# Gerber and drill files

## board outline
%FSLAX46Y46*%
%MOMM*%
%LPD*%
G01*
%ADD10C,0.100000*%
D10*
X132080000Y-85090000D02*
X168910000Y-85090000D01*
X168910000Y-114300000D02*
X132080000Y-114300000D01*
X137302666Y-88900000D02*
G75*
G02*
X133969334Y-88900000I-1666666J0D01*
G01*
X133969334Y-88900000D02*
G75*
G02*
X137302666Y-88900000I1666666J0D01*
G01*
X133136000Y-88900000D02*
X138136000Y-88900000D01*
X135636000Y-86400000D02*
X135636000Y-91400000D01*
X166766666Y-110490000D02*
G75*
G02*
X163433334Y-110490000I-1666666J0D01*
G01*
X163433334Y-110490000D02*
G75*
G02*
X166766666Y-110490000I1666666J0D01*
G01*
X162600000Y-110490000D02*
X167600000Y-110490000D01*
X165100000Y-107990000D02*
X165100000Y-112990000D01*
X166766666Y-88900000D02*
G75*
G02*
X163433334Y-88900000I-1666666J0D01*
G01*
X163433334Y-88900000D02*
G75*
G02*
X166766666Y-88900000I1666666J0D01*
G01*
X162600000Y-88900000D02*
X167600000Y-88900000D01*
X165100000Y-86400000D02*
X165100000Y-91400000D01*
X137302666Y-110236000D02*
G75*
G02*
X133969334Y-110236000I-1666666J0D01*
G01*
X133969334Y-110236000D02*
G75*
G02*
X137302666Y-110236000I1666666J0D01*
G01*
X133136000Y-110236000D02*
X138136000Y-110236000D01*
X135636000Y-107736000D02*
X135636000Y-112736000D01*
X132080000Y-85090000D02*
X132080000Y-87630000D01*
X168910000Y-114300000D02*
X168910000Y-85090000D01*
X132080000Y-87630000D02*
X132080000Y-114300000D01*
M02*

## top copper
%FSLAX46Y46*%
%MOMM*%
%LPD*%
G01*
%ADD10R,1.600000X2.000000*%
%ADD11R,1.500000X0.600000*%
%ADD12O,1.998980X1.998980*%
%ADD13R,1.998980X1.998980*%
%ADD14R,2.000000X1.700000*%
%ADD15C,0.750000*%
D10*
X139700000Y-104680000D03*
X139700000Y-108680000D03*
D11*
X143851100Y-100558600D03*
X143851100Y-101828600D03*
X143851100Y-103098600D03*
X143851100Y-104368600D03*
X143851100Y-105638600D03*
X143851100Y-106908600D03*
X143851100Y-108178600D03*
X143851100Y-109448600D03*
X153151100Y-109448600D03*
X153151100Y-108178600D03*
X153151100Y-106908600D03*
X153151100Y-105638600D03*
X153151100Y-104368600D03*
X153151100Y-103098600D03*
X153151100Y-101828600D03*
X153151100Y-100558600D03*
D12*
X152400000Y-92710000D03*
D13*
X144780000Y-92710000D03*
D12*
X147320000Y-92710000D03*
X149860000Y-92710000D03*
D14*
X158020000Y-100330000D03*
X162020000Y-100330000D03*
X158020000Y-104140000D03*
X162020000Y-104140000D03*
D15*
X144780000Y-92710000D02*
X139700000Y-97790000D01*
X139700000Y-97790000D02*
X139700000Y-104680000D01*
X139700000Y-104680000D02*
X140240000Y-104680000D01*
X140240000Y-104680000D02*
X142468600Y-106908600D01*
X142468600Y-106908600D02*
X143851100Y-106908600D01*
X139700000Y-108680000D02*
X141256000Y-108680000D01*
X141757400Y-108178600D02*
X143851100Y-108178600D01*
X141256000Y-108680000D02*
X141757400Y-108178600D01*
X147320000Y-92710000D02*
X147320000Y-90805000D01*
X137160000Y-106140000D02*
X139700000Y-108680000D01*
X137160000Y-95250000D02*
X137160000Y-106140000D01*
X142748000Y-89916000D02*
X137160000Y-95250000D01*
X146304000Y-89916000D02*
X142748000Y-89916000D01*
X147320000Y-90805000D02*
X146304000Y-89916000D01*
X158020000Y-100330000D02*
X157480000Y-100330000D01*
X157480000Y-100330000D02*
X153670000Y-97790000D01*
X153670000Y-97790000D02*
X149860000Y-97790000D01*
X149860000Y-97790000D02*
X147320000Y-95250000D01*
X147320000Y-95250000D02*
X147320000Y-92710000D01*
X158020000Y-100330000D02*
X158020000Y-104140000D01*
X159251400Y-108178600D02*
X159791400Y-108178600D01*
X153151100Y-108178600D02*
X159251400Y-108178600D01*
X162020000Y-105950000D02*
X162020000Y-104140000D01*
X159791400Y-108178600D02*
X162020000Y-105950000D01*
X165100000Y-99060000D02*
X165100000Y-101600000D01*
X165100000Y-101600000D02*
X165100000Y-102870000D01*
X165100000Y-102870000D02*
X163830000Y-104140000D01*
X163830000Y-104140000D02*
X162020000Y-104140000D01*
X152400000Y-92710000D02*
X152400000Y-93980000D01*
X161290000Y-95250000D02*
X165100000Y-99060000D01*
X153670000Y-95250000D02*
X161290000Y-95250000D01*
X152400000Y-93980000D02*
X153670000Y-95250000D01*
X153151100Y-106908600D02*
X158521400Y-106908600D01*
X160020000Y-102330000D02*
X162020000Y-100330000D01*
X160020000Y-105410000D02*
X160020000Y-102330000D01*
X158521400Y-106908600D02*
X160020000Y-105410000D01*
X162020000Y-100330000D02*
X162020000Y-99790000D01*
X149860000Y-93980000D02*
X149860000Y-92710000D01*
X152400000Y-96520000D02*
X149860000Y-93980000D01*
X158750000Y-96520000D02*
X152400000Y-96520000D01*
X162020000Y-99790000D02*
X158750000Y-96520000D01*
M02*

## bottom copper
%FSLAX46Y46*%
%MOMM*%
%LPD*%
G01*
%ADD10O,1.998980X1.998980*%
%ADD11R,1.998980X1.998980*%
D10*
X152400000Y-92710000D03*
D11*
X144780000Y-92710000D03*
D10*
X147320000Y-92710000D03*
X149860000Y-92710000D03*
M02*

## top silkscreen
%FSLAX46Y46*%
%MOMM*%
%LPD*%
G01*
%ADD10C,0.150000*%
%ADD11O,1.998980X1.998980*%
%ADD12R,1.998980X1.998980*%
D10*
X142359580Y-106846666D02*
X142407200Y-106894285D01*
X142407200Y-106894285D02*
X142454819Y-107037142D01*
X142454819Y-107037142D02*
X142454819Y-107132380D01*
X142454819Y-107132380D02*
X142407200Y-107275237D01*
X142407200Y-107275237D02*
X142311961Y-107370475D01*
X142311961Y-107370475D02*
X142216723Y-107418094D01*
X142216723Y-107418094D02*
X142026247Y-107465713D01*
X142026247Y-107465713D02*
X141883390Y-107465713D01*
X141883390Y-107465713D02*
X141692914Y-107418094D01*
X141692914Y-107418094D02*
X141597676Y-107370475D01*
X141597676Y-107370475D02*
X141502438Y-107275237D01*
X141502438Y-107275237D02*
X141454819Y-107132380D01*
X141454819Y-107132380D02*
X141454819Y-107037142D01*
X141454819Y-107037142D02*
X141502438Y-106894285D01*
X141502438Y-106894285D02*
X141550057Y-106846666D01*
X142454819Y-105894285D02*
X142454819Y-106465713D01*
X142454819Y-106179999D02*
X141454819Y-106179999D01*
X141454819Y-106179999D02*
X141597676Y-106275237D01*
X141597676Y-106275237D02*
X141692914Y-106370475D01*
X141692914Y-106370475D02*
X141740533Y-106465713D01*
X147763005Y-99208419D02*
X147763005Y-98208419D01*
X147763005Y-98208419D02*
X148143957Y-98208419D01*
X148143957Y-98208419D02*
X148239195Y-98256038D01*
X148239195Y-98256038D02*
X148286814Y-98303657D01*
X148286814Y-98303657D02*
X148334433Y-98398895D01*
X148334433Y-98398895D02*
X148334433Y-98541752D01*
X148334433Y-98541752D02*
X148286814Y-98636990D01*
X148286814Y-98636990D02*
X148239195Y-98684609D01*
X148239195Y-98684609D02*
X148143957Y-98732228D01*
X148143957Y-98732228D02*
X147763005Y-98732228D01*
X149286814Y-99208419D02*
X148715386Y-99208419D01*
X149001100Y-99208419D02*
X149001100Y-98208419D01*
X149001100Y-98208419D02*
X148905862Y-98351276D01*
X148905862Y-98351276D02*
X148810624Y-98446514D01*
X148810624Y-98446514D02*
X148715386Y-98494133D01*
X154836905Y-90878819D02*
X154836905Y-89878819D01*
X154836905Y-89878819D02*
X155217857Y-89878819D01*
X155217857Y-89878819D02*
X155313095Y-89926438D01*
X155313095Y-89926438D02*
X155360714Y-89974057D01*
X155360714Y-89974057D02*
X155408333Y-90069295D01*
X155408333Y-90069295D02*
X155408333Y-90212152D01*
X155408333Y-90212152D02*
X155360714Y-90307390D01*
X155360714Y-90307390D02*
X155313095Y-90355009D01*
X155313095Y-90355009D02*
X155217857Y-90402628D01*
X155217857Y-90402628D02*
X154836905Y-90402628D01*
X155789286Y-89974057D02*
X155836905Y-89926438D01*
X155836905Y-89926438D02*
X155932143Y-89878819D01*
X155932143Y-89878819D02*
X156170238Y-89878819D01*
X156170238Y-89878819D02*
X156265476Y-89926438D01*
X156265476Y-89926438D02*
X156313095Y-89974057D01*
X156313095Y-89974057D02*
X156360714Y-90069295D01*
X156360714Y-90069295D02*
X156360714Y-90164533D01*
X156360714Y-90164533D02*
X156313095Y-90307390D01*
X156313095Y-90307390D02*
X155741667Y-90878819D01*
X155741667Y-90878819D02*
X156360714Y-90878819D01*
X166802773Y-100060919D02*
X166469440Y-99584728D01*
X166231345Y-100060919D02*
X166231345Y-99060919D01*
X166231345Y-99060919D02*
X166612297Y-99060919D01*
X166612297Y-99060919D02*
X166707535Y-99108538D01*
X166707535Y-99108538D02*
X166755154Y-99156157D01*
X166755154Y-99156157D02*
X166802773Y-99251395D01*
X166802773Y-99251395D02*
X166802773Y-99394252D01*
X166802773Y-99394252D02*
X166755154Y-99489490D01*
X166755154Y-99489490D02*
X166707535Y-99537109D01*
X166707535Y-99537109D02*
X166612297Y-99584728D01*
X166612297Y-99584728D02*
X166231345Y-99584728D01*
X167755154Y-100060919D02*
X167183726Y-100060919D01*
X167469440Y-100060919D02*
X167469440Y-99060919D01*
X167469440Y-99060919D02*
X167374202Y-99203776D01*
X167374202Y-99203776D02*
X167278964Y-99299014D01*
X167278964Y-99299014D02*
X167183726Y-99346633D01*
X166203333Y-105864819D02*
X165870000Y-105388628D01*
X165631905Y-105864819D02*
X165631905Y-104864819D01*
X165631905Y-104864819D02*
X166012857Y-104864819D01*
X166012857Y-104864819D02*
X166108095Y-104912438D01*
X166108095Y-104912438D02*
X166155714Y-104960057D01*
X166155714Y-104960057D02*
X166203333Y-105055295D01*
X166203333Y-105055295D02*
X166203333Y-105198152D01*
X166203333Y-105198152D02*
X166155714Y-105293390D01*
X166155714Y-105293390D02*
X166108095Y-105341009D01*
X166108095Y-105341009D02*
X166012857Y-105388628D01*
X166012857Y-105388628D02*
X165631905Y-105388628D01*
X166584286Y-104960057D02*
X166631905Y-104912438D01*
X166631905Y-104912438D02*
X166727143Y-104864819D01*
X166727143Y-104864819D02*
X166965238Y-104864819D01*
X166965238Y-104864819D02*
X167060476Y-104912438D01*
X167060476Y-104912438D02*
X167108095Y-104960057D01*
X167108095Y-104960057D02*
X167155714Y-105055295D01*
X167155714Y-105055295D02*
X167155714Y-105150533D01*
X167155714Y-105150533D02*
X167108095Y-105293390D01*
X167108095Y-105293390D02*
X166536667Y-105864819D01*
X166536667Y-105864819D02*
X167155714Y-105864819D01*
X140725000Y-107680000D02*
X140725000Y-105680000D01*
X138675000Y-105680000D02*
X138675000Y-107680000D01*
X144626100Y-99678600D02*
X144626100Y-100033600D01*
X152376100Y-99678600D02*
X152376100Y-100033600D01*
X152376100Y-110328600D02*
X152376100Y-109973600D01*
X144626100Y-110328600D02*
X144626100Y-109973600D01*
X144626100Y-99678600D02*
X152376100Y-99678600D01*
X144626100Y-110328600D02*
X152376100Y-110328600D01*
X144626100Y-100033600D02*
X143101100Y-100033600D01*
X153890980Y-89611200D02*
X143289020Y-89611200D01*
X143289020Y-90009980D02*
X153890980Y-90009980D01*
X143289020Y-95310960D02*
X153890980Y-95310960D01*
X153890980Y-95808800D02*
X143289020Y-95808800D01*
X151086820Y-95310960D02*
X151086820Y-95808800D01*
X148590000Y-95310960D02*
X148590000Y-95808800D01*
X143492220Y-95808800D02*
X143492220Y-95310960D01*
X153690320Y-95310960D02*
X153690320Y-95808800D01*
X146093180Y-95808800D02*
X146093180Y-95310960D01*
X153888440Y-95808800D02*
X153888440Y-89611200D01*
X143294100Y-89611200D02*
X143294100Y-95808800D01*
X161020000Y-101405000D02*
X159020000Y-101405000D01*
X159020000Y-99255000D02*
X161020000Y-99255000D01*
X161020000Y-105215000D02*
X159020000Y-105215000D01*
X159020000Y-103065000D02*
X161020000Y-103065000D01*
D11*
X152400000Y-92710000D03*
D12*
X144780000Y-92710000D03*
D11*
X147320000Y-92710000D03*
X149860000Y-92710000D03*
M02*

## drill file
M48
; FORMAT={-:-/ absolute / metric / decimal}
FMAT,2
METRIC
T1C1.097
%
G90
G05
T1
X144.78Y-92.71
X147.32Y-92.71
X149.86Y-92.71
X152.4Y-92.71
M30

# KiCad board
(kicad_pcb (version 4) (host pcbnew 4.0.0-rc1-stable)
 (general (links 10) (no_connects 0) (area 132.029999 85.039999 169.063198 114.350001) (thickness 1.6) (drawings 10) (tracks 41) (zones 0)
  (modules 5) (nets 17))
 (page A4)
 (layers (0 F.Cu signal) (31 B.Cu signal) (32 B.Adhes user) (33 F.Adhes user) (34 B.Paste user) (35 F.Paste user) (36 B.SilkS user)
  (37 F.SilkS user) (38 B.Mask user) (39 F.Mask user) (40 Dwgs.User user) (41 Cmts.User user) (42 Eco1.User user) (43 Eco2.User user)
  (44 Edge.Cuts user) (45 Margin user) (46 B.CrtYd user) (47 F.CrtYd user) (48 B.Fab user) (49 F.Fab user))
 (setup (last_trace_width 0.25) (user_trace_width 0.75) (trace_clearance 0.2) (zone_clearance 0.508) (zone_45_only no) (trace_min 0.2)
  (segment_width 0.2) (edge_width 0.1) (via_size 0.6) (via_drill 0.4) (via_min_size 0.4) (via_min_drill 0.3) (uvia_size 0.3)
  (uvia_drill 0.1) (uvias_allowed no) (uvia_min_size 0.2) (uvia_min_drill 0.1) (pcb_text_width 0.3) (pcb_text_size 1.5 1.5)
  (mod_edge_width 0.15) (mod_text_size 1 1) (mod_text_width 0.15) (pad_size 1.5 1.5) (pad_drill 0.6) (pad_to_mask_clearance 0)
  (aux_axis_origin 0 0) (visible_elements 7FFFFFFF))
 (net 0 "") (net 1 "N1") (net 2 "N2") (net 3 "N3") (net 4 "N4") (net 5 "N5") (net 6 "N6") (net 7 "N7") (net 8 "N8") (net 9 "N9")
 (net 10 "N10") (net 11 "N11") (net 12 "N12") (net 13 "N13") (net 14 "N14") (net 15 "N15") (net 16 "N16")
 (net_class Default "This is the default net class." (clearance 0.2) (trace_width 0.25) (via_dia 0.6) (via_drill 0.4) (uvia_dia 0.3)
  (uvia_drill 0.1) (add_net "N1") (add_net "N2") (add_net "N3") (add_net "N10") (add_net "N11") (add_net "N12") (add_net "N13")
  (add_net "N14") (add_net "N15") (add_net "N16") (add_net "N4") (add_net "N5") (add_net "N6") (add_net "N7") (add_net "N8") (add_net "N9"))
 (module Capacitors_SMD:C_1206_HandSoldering (layer F.Cu) (at 139.7 106.68 270)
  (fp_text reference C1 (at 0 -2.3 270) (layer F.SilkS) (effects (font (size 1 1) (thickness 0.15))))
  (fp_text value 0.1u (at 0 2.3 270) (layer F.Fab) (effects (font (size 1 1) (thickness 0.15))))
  (fp_line (start 1 -1.025) (end -1 -1.025) (layer F.SilkS) (width 0.15))
  (fp_line (start -1 1.025) (end 1 1.025) (layer F.SilkS) (width 0.15))
  (pad 1 smd rect (at -2 0 270) (size 2 1.6) (layers F.Cu F.Paste F.Mask) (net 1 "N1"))
  (pad 2 smd rect (at 2 0 270) (size 2 1.6) (layers F.Cu F.Paste F.Mask) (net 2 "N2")))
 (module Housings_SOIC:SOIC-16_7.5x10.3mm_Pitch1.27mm (layer F.Cu) (at 148.5011 105.0036)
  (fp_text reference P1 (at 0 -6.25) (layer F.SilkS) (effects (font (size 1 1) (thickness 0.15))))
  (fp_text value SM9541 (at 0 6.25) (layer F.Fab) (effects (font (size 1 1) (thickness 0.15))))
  (fp_line (start -3.875 -5.325) (end -3.875 -4.97) (layer F.SilkS) (width 0.15))
  (fp_line (start 3.875 -5.325) (end 3.875 -4.97) (layer F.SilkS) (width 0.15))
  (fp_line (start 3.875 5.325) (end 3.875 4.97) (layer F.SilkS) (width 0.15))
  (fp_line (start -3.875 5.325) (end -3.875 4.97) (layer F.SilkS) (width 0.15))
  (fp_line (start -3.875 -5.325) (end 3.875 -5.325) (layer F.SilkS) (width 0.15))
  (fp_line (start -3.875 5.325) (end 3.875 5.325) (layer F.SilkS) (width 0.15))
  (fp_line (start -3.875 -4.97) (end -5.4 -4.97) (layer F.SilkS) (width 0.15))
  (pad 1 smd rect (at -4.65 -4.445) (size 1.5 0.6) (layers F.Cu F.Paste F.Mask) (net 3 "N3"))
  (pad 2 smd rect (at -4.65 -3.175) (size 1.5 0.6) (layers F.Cu F.Paste F.Mask) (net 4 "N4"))
  (pad 3 smd rect (at -4.65 -1.905) (size 1.5 0.6) (layers F.Cu F.Paste F.Mask) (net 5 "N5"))
  (pad 4 smd rect (at -4.65 -0.635) (size 1.5 0.6) (layers F.Cu F.Paste F.Mask) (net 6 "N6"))
  (pad 5 smd rect (at -4.65 0.635) (size 1.5 0.6) (layers F.Cu F.Paste F.Mask) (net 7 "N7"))
  (pad 6 smd rect (at -4.65 1.905) (size 1.5 0.6) (layers F.Cu F.Paste F.Mask) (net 1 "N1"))
  (pad 7 smd rect (at -4.65 3.175) (size 1.5 0.6) (layers F.Cu F.Paste F.Mask) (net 2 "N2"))
  (pad 8 smd rect (at -4.65 4.445) (size 1.5 0.6) (layers F.Cu F.Paste F.Mask) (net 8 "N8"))
  (pad 9 smd rect (at 4.65 4.445) (size 1.5 0.6) (layers F.Cu F.Paste F.Mask) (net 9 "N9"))
  (pad 10 smd rect (at 4.65 3.175) (size 1.5 0.6) (layers F.Cu F.Paste F.Mask) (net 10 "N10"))
  (pad 11 smd rect (at 4.65 1.905) (size 1.5 0.6) (layers F.Cu F.Paste F.Mask) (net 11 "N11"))
  (pad 12 smd rect (at 4.65 0.635) (size 1.5 0.6) (layers F.Cu F.Paste F.Mask) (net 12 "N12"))
  (pad 13 smd rect (at 4.65 -0.635) (size 1.5 0.6) (layers F.Cu F.Paste F.Mask) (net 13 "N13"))
  (pad 14 smd rect (at 4.65 -1.905) (size 1.5 0.6) (layers F.Cu F.Paste F.Mask) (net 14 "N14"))
  (pad 15 smd rect (at 4.65 -3.175) (size 1.5 0.6) (layers F.Cu F.Paste F.Mask) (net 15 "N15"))
  (pad 16 smd rect (at 4.65 -4.445) (size 1.5 0.6) (layers F.Cu F.Paste F.Mask) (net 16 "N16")))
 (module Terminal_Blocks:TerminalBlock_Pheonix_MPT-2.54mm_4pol (layer F.Cu) (at 144.78 92.71)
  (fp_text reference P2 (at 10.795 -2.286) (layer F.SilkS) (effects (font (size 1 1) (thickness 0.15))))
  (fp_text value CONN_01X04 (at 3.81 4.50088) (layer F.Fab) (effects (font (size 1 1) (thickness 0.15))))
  (fp_line (start 9.11098 -3.0988) (end -1.49098 -3.0988) (layer F.SilkS) (width 0.15))
  (fp_line (start -1.49098 -2.70002) (end 9.11098 -2.70002) (layer F.SilkS) (width 0.15))
  (fp_line (start -1.49098 2.60096) (end 9.11098 2.60096) (layer F.SilkS) (width 0.15))
  (fp_line (start 9.11098 3.0988) (end -1.49098 3.0988) (layer F.SilkS) (width 0.15))
  (fp_line (start 6.30682 2.60096) (end 6.30682 3.0988) (layer F.SilkS) (width 0.15))
  (fp_line (start 3.81 2.60096) (end 3.81 3.0988) (layer F.SilkS) (width 0.15))
  (fp_line (start -1.28778 3.0988) (end -1.28778 2.60096) (layer F.SilkS) (width 0.15))
  (fp_line (start 8.91032 2.60096) (end 8.91032 3.0988) (layer F.SilkS) (width 0.15))
  (fp_line (start 1.31318 3.0988) (end 1.31318 2.60096) (layer F.SilkS) (width 0.15))
  (fp_line (start 9.10844 3.0988) (end 9.10844 -3.0988) (layer F.SilkS) (width 0.15))
  (fp_line (start -1.4859 -3.0988) (end -1.4859 3.0988) (layer F.SilkS) (width 0.15))
  (pad 4 thru_hole oval (at 7.62 0 180) (size 1.99898 1.99898) (drill 1.09728) (layers *.Cu *.Mask F.SilkS) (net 10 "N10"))
  (pad 1 thru_hole rect (at 0 0 180) (size 1.99898 1.99898) (drill 1.09728) (layers *.Cu *.Mask F.SilkS) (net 1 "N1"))
  (pad 2 thru_hole oval (at 2.54 0 180) (size 1.99898 1.99898) (drill 1.09728) (layers *.Cu *.Mask F.SilkS) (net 2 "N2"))
  (pad 3 thru_hole oval (at 5.08 0 180) (size 1.99898 1.99898) (drill 1.09728) (layers *.Cu *.Mask F.SilkS) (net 11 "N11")))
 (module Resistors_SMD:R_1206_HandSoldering (layer F.Cu) (at 160.02 100.33)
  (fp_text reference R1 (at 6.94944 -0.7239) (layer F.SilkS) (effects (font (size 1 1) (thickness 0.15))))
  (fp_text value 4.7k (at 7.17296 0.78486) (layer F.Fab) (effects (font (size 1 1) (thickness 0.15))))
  (fp_line (start 1 1.075) (end -1 1.075) (layer F.SilkS) (width 0.15))
  (fp_line (start -1 -1.075) (end 1 -1.075) (layer F.SilkS) (width 0.15))
  (pad 1 smd rect (at -2 0) (size 2 1.7) (layers F.Cu F.Paste F.Mask) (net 2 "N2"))
  (pad 2 smd rect (at 2 0) (size 2 1.7) (layers F.Cu F.Paste F.Mask) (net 11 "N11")))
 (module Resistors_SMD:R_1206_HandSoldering (layer F.Cu) (at 160.02 104.14)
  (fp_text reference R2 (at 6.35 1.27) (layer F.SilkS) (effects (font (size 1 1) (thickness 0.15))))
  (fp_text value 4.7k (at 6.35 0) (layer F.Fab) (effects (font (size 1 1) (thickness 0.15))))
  (fp_line (start 1 1.075) (end -1 1.075) (layer F.SilkS) (width 0.15))
  (fp_line (start -1 -1.075) (end 1 -1.075) (layer F.SilkS) (width 0.15))
  (pad 1 smd rect (at -2 0) (size 2 1.7) (layers F.Cu F.Paste F.Mask) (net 2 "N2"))
  (pad 2 smd rect (at 2 0) (size 2 1.7) (layers F.Cu F.Paste F.Mask) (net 10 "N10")))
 (gr_line (start 132.08 85.09) (end 168.91 85.09) (angle 90) (layer Edge.Cuts) (width 0.1))
 (gr_line (start 168.91 114.3) (end 132.08 114.3) (angle 90) (layer Edge.Cuts) (width 0.1))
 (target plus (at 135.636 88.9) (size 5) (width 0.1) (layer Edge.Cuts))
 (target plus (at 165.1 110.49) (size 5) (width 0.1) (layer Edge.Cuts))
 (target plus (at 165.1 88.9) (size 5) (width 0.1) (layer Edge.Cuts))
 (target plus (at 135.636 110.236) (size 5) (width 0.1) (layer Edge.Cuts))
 (gr_line (start 132.08 85.09) (end 132.08 87.63) (angle 90) (layer Edge.Cuts) (width 0.1))
 (gr_line (start 168.91 114.3) (end 168.91 85.09) (angle 90) (layer Edge.Cuts) (width 0.1))
 (gr_line (start 132.08 87.63) (end 132.08 114.3) (angle 90) (layer Edge.Cuts) (width 0.1))
 (segment (start 144.78 92.71) (end 139.7 97.79) (width 0.75) (layer F.Cu) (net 1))
 (segment (start 139.7 97.79) (end 139.7 104.68) (width 0.75) (layer F.Cu) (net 1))
 (segment (start 139.7 104.68) (end 140.24 104.68) (width 0.75) (layer F.Cu) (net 1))
 (segment (start 140.24 104.68) (end 142.4686 106.9086) (width 0.75) (layer F.Cu) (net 1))
 (segment (start 142.4686 106.9086) (end 143.8511 106.9086) (width 0.75) (layer F.Cu) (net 1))
 (segment (start 139.7 108.68) (end 141.256 108.68) (width 0.75) (layer F.Cu) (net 2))
 (segment (start 141.7574 108.1786) (end 143.8511 108.1786) (width 0.75) (layer F.Cu) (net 2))
 (segment (start 141.256 108.68) (end 141.7574 108.1786) (width 0.75) (layer F.Cu) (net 2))
 (segment (start 147.32 92.71) (end 147.32 90.805) (width 0.75) (layer F.Cu) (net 2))
 (segment (start 137.16 106.14) (end 139.7 108.68) (width 0.75) (layer F.Cu) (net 2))
 (segment (start 137.16 95.25) (end 137.16 106.14) (width 0.75) (layer F.Cu) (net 2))
 (segment (start 142.748 89.916) (end 137.16 95.25) (width 0.75) (layer F.Cu) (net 2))
 (segment (start 146.304 89.916) (end 142.748 89.916) (width 0.75) (layer F.Cu) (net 2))
 (segment (start 147.32 90.805) (end 146.304 89.916) (width 0.75) (layer F.Cu) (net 2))
 (segment (start 158.02 100.33) (end 157.48 100.33) (width 0.75) (layer F.Cu) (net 2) (status 30))
 (segment (start 157.48 100.33) (end 153.67 97.79) (width 0.75) (layer F.Cu) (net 2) (status 10))
 (segment (start 153.67 97.79) (end 149.86 97.79) (width 0.75) (layer F.Cu) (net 2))
 (segment (start 149.86 97.79) (end 147.32 95.25) (width 0.75) (layer F.Cu) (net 2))
 (segment (start 147.32 95.25) (end 147.32 92.71) (width 0.75) (layer F.Cu) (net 2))
 (segment (start 158.02 100.33) (end 158.02 104.14) (width 0.75) (layer F.Cu) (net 2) (status 20))
 (segment (start 159.2514 108.1786) (end 159.7914 108.1786) (width 0.75) (layer F.Cu) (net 10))
 (segment (start 153.1511 108.1786) (end 159.2514 108.1786) (width 0.75) (layer F.Cu) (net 10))
 (segment (start 162.02 105.95) (end 162.02 104.14) (width 0.75) (layer F.Cu) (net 10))
 (segment (start 159.7914 108.1786) (end 162.02 105.95) (width 0.75) (layer F.Cu) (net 10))
 (segment (start 165.1 99.06) (end 165.1 101.6) (width 0.75) (layer F.Cu) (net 10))
 (segment (start 165.1 101.6) (end 165.1 102.87) (width 0.75) (layer F.Cu) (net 10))
 (segment (start 165.1 102.87) (end 163.83 104.14) (width 0.75) (layer F.Cu) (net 10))
 (segment (start 163.83 104.14) (end 162.02 104.14) (width 0.75) (layer F.Cu) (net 10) (status 20))
 (segment (start 152.4 92.71) (end 152.4 93.98) (width 0.75) (layer F.Cu) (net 10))
 (segment (start 161.29 95.25) (end 165.1 99.06) (width 0.75) (layer F.Cu) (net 10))
 (segment (start 153.67 95.25) (end 161.29 95.25) (width 0.75) (layer F.Cu) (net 10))
 (segment (start 152.4 93.98) (end 153.67 95.25) (width 0.75) (layer F.Cu) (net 10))
 (segment (start 153.1511 106.9086) (end 158.5214 106.9086) (width 0.75) (layer F.Cu) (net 11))
 (segment (start 160.02 102.33) (end 162.02 100.33) (width 0.75) (layer F.Cu) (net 11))
 (segment (start 160.02 105.41) (end 160.02 102.33) (width 0.75) (layer F.Cu) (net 11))
 (segment (start 158.5214 106.9086) (end 160.02 105.41) (width 0.75) (layer F.Cu) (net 11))
 (segment (start 162.02 100.33) (end 162.02 99.79) (width 0.75) (layer F.Cu) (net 11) (status 10))
 (segment (start 149.86 93.98) (end 149.86 92.71) (width 0.75) (layer F.Cu) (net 11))
 (segment (start 152.4 96.52) (end 149.86 93.98) (width 0.75) (layer F.Cu) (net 11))
 (segment (start 158.75 96.52) (end 152.4 96.52) (width 0.75) (layer F.Cu) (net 11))
 (segment (start 162.02 99.79) (end 158.75 96.52) (width 0.75) (layer F.Cu) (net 11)))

